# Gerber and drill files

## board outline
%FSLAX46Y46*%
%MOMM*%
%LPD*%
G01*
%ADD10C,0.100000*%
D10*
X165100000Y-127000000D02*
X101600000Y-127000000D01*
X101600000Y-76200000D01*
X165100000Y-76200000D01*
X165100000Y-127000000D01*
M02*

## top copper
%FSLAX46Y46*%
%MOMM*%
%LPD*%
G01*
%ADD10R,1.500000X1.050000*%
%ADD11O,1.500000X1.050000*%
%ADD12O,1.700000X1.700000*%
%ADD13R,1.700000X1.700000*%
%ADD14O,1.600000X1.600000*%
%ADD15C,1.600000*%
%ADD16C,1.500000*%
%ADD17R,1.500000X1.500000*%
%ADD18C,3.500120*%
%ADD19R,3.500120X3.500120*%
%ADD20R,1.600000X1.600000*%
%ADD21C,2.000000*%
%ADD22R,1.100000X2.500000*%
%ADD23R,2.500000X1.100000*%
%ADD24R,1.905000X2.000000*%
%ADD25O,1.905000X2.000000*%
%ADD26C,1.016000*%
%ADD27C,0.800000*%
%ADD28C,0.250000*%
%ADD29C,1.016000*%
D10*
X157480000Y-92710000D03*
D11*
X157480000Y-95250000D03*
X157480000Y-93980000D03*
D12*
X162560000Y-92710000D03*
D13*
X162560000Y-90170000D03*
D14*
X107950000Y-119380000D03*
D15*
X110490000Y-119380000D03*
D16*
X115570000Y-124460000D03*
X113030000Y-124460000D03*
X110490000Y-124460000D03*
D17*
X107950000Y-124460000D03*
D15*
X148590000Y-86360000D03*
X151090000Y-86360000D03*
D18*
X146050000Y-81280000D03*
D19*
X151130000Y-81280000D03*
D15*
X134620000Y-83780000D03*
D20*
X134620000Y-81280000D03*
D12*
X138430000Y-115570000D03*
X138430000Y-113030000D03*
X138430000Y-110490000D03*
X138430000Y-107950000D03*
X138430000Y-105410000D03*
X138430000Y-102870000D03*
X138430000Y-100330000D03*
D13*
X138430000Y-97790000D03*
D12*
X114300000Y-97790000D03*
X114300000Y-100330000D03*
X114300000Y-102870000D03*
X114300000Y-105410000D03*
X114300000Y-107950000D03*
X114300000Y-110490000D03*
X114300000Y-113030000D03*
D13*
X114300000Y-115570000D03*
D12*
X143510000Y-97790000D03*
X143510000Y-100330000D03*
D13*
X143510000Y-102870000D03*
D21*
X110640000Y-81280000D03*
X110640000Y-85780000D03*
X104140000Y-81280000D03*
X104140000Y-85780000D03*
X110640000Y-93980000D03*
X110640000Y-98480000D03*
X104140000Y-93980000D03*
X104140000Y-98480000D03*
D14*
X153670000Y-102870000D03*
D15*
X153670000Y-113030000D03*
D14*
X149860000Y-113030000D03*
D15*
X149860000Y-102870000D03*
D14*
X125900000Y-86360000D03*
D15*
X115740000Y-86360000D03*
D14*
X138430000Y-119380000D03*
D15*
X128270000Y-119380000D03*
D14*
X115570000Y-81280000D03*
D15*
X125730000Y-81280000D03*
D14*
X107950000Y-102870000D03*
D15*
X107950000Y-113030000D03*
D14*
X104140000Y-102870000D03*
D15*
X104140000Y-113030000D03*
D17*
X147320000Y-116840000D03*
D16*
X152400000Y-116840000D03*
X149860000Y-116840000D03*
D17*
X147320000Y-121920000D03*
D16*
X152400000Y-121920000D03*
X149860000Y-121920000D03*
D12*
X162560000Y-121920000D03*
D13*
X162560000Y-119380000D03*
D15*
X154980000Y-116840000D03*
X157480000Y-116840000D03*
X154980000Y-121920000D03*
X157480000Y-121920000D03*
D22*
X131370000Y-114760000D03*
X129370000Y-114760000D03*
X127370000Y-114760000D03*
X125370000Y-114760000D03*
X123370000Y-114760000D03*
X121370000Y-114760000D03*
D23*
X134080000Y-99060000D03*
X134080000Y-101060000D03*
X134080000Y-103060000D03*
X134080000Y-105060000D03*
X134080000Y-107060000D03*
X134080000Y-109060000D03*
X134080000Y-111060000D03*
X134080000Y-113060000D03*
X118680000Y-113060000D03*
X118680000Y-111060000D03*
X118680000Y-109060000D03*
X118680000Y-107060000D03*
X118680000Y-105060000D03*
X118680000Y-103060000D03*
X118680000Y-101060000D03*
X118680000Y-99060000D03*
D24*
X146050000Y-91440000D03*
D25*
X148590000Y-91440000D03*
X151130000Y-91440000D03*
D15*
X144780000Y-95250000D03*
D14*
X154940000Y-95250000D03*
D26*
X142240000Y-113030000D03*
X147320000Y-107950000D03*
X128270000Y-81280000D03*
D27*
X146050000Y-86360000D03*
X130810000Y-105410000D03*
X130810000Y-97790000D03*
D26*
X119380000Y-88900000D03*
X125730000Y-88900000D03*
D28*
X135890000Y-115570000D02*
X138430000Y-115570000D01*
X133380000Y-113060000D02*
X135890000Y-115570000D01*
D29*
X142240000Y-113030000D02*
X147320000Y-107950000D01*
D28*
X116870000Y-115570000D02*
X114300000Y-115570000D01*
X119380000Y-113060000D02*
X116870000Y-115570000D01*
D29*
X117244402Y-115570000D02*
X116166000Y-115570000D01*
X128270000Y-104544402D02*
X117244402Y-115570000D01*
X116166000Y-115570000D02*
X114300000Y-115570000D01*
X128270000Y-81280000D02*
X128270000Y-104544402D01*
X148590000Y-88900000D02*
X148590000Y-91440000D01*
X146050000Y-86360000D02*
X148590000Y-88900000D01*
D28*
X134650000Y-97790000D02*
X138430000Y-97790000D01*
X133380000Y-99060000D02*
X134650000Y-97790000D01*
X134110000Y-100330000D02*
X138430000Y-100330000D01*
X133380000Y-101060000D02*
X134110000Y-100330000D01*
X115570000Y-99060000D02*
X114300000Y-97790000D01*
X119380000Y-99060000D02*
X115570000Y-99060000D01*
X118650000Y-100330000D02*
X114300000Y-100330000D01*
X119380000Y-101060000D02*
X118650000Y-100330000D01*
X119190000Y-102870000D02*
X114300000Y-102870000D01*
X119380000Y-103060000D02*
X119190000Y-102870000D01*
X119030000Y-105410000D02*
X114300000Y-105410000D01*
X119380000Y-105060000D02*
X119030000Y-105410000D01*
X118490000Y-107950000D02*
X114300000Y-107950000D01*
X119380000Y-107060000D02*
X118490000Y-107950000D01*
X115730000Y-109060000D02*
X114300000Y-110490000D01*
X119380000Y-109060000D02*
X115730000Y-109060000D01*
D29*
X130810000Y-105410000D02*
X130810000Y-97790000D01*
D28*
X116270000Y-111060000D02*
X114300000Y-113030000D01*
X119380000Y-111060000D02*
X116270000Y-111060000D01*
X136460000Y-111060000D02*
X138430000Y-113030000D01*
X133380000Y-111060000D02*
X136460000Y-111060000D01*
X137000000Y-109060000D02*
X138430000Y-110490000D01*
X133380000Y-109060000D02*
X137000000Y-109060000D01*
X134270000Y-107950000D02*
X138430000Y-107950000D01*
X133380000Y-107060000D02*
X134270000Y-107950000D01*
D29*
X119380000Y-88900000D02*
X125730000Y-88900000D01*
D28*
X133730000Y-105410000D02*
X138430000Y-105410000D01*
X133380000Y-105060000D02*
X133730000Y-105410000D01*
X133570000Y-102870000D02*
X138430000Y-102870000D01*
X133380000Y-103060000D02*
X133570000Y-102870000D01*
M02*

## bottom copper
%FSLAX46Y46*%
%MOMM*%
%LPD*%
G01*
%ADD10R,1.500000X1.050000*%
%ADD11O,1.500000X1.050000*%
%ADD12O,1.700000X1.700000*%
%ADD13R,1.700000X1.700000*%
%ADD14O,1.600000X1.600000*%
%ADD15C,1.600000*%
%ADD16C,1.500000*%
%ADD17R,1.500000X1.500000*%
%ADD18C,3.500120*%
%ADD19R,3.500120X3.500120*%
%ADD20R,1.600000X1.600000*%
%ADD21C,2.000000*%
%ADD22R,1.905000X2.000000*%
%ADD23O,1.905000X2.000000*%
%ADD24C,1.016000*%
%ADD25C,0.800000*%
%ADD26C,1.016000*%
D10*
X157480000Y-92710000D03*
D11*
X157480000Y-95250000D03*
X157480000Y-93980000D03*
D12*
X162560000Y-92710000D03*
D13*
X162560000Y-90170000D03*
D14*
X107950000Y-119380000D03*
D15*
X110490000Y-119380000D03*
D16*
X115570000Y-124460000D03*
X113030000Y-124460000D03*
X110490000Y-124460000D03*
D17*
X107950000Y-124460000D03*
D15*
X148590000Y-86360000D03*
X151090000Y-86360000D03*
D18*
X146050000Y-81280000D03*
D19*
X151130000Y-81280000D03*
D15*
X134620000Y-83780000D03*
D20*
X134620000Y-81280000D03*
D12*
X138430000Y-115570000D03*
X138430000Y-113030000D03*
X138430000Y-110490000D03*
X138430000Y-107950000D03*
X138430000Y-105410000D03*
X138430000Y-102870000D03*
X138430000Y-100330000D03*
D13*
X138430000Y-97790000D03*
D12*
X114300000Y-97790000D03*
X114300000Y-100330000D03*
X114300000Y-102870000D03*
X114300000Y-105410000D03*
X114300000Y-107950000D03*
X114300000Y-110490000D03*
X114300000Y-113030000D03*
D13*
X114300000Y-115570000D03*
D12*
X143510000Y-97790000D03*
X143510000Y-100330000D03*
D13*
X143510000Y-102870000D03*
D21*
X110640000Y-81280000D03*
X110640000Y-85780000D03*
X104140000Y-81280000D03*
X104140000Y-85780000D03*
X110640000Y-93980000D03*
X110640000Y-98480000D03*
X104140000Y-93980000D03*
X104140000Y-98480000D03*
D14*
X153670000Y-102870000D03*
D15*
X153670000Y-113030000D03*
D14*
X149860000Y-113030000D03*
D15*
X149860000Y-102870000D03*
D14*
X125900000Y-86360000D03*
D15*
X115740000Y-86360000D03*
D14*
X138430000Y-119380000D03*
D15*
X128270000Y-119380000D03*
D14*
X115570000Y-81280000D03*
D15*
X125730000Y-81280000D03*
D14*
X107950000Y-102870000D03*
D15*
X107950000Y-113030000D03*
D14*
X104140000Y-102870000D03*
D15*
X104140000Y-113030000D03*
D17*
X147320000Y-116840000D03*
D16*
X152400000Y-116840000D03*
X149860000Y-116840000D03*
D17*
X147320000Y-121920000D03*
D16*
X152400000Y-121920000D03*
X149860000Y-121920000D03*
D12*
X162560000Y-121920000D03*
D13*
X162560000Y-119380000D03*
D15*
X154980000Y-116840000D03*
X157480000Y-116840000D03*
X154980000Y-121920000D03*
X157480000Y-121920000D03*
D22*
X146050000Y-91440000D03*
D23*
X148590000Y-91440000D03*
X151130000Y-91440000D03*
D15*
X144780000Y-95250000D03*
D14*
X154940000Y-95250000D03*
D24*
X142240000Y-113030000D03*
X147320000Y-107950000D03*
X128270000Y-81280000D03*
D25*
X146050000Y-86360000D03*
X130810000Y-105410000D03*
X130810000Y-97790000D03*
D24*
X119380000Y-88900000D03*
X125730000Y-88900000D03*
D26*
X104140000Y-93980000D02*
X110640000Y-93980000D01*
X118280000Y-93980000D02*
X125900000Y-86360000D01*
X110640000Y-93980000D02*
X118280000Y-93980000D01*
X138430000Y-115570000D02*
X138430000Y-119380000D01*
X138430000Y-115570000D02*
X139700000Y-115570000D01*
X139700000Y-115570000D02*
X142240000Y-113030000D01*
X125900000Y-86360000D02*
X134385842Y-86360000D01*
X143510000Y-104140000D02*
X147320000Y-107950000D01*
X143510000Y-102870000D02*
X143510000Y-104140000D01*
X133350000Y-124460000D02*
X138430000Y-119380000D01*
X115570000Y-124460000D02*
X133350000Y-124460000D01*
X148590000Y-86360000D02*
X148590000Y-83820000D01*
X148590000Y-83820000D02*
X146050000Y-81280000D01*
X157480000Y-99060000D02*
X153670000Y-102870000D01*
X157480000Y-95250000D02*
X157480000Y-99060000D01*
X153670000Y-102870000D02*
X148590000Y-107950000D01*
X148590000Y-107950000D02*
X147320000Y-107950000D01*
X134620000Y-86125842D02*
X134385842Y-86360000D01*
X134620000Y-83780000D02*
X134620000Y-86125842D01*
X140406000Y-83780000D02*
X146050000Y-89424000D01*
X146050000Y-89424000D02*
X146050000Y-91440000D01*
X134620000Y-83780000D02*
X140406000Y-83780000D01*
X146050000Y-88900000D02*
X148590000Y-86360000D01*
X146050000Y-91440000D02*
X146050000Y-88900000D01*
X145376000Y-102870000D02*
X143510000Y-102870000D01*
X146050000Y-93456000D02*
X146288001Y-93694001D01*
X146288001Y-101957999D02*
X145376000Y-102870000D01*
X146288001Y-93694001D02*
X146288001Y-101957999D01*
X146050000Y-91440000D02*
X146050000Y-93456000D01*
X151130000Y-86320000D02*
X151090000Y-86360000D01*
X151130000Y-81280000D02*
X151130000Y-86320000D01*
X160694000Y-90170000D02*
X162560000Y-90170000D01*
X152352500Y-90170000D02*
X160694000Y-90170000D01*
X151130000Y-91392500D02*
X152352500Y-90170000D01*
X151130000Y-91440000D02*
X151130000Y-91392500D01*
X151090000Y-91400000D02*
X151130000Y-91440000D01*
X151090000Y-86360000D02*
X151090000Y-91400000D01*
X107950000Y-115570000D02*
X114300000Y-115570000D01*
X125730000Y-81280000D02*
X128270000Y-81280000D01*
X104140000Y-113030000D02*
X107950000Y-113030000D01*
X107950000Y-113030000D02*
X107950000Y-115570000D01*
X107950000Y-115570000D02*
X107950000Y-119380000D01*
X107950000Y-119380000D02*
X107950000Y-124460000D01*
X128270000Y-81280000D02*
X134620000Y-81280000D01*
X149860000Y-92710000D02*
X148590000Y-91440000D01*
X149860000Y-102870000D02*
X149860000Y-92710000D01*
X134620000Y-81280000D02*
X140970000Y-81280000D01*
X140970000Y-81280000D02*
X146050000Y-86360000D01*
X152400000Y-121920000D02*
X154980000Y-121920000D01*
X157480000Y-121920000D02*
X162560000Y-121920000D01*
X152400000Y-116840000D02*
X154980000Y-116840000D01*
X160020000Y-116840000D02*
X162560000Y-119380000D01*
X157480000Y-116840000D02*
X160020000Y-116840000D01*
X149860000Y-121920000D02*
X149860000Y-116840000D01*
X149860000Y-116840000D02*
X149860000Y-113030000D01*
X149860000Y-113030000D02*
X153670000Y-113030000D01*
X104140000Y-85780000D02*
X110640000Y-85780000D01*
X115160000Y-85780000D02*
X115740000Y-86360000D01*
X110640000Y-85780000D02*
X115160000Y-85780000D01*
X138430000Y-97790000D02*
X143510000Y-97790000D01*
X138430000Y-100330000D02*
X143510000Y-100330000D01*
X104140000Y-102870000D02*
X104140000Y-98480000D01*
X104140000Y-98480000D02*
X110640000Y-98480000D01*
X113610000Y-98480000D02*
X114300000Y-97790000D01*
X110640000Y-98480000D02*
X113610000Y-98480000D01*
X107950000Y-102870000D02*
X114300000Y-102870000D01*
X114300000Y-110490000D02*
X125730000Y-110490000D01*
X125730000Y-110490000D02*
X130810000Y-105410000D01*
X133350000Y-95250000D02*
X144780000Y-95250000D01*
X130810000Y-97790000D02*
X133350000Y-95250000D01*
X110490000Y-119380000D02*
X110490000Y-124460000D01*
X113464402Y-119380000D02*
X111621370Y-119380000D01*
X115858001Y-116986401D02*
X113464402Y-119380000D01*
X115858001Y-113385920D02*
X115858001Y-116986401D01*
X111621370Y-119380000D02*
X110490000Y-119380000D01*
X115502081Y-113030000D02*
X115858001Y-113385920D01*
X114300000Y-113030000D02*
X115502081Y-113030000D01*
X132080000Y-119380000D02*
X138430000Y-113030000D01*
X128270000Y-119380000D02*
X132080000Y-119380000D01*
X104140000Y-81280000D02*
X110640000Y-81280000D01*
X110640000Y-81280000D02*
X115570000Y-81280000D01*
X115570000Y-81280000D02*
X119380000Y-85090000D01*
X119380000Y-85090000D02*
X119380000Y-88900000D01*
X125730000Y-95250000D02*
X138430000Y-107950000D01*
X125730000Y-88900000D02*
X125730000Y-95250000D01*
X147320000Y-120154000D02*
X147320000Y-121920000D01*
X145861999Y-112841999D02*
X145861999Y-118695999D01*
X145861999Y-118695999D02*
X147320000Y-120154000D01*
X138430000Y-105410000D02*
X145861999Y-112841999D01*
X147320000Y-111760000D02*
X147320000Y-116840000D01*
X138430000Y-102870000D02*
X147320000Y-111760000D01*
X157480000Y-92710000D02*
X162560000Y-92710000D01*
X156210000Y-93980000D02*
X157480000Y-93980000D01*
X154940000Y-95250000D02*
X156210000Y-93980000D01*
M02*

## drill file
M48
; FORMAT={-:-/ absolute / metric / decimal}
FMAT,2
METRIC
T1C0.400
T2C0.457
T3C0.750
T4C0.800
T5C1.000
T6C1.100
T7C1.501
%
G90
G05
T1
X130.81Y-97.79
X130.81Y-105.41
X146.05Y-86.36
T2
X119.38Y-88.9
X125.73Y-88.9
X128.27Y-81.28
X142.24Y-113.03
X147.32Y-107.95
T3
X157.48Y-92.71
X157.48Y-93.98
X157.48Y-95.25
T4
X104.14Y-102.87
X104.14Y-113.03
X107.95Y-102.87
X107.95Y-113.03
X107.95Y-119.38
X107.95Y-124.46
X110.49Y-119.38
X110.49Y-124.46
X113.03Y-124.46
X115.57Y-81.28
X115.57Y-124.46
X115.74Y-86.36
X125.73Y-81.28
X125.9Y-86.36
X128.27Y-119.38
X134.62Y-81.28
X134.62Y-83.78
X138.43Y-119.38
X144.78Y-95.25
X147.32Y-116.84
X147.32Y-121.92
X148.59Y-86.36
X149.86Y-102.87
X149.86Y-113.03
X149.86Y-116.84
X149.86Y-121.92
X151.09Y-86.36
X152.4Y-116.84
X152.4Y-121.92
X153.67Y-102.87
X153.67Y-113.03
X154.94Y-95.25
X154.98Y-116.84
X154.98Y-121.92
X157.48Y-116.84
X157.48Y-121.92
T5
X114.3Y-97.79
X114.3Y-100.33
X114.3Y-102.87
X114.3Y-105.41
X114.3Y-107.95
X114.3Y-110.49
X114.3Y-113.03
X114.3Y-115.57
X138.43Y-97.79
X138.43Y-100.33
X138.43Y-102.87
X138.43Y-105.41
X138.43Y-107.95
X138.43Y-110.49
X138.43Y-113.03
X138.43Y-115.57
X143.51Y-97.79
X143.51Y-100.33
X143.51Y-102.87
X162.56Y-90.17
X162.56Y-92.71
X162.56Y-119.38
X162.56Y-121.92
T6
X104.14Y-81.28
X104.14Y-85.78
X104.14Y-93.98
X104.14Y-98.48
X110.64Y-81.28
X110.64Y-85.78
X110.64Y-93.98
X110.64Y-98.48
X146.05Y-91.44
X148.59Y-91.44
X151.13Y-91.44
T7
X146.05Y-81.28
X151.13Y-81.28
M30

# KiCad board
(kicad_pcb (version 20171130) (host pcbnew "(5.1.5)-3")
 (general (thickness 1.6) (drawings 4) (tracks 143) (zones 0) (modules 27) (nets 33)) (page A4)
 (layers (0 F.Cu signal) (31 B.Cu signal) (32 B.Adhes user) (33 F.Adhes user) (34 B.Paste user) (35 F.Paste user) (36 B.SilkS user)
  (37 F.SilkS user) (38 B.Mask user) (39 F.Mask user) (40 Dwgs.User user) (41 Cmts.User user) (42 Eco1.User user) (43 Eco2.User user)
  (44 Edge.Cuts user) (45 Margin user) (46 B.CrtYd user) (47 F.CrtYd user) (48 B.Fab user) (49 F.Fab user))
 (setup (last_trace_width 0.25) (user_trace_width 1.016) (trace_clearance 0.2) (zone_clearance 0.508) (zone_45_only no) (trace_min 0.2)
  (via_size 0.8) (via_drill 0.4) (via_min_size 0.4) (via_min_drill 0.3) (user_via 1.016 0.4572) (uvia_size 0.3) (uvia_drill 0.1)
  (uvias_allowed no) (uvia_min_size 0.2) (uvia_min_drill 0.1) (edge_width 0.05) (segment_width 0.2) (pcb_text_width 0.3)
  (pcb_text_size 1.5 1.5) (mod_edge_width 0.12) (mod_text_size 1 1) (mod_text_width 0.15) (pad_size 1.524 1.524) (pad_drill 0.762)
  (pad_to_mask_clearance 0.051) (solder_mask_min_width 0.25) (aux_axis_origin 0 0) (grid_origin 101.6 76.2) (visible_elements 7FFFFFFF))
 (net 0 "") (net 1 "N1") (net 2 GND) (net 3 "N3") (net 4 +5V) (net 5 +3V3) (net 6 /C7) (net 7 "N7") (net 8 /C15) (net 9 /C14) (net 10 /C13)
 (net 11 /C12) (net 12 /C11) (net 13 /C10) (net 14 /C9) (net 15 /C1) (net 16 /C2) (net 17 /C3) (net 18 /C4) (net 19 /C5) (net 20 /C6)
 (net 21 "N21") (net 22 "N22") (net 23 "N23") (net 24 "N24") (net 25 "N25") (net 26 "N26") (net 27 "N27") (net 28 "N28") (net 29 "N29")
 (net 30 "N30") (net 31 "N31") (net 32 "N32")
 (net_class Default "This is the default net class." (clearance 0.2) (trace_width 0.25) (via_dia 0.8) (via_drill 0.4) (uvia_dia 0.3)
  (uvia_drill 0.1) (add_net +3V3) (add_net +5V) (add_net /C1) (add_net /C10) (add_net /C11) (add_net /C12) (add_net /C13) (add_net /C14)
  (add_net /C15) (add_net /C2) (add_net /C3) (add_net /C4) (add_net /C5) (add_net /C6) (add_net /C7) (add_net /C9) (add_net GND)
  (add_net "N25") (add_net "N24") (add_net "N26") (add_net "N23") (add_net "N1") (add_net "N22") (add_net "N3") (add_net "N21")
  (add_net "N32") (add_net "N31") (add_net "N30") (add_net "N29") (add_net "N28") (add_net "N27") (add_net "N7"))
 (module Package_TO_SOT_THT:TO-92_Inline (layer F.Cu) (at 157.48 92.71 270)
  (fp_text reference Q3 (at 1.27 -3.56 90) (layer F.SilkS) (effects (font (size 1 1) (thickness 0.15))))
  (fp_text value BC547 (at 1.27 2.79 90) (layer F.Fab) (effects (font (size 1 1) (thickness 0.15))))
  (pad 1 thru_hole rect (at 0 0 270) (size 1.05 1.5) (drill 0.75) (layers *.Cu *.Mask) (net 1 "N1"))
  (pad 3 thru_hole oval (at 2.54 0 270) (size 1.05 1.5) (drill 0.75) (layers *.Cu *.Mask) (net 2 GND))
  (pad 2 thru_hole oval (at 1.27 0 270) (size 1.05 1.5) (drill 0.75) (layers *.Cu *.Mask) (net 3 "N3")))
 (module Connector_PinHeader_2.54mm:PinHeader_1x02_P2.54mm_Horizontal (layer F.Cu) (at 162.56 90.17)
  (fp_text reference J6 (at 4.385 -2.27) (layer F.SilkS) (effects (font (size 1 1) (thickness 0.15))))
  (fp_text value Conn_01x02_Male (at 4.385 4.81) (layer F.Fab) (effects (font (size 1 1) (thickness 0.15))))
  (pad 2 thru_hole oval (at 0 2.54) (size 1.7 1.7) (drill 1) (layers *.Cu *.Mask) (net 1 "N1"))
  (pad 1 thru_hole rect (at 0 0) (size 1.7 1.7) (drill 1) (layers *.Cu *.Mask) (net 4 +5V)))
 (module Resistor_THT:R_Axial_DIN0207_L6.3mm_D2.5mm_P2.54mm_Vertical (layer F.Cu) (at 110.49 119.38 180)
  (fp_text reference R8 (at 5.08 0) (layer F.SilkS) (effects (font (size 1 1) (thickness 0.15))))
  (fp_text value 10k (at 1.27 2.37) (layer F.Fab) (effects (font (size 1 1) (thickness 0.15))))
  (pad 2 thru_hole oval (at 2.54 0 180) (size 1.6 1.6) (drill 0.8) (layers *.Cu *.Mask) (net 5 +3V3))
  (pad 1 thru_hole circle (at 0 0 180) (size 1.6 1.6) (drill 0.8) (layers *.Cu *.Mask) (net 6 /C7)))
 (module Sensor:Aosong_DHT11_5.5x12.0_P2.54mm (layer F.Cu) (at 107.95 124.46 90)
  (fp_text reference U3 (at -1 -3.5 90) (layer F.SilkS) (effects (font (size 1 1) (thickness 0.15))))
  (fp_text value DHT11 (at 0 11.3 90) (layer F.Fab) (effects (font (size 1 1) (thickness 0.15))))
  (pad 4 thru_hole circle (at 0 7.62 90) (size 1.5 1.5) (drill 0.8) (layers *.Cu *.Mask) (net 2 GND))
  (pad 3 thru_hole circle (at 0 5.08 90) (size 1.5 1.5) (drill 0.8) (layers *.Cu *.Mask) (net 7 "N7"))
  (pad 2 thru_hole circle (at 0 2.54 90) (size 1.5 1.5) (drill 0.8) (layers *.Cu *.Mask) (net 6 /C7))
  (pad 1 thru_hole rect (at 0 0 90) (size 1.5 1.5) (drill 0.8) (layers *.Cu *.Mask) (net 5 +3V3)))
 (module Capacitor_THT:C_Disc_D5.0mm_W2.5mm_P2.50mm (layer F.Cu) (at 151.09 86.36 180)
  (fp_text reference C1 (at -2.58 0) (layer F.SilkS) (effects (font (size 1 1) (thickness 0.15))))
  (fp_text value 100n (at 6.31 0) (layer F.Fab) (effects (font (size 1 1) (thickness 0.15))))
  (pad 2 thru_hole circle (at 2.5 0 180) (size 1.6 1.6) (drill 0.8) (layers *.Cu *.Mask) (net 2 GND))
  (pad 1 thru_hole circle (at 0 0 180) (size 1.6 1.6) (drill 0.8) (layers *.Cu *.Mask) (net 4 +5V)))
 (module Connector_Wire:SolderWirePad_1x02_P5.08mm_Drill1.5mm (layer F.Cu) (at 151.13 81.28 180)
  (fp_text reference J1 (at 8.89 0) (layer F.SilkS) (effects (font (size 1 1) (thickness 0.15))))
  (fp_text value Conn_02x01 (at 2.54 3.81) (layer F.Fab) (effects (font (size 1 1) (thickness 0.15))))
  (pad 2 thru_hole circle (at 5.08 0 180) (size 3.50012 3.50012) (drill 1.50114) (layers *.Cu *.Mask) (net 2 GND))
  (pad 1 thru_hole rect (at 0 0 180) (size 3.50012 3.50012) (drill 1.50114) (layers *.Cu *.Mask) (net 4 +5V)))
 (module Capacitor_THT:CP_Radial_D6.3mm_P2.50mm (layer F.Cu) (at 134.62 81.28 270)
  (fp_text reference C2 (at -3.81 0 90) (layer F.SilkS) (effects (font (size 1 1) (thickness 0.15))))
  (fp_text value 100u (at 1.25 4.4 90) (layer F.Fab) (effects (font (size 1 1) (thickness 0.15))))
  (pad 2 thru_hole circle (at 2.5 0 270) (size 1.6 1.6) (drill 0.8) (layers *.Cu *.Mask) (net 2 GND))
  (pad 1 thru_hole rect (at 0 0 270) (size 1.6 1.6) (drill 0.8) (layers *.Cu *.Mask) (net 5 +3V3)))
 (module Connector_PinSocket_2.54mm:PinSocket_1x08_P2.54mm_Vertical (layer F.Cu) (at 138.43 97.79)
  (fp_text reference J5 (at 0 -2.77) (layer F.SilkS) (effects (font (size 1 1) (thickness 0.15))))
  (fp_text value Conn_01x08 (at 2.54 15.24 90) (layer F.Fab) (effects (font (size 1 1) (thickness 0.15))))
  (pad 8 thru_hole oval (at 0 17.78) (size 1.7 1.7) (drill 1) (layers *.Cu *.Mask) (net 2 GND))
  (pad 7 thru_hole oval (at 0 15.24) (size 1.7 1.7) (drill 1) (layers *.Cu *.Mask) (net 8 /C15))
  (pad 6 thru_hole oval (at 0 12.7) (size 1.7 1.7) (drill 1) (layers *.Cu *.Mask) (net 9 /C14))
  (pad 5 thru_hole oval (at 0 10.16) (size 1.7 1.7) (drill 1) (layers *.Cu *.Mask) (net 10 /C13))
  (pad 4 thru_hole oval (at 0 7.62) (size 1.7 1.7) (drill 1) (layers *.Cu *.Mask) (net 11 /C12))
  (pad 3 thru_hole oval (at 0 5.08) (size 1.7 1.7) (drill 1) (layers *.Cu *.Mask) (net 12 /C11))
  (pad 2 thru_hole oval (at 0 2.54) (size 1.7 1.7) (drill 1) (layers *.Cu *.Mask) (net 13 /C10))
  (pad 1 thru_hole rect (at 0 0) (size 1.7 1.7) (drill 1) (layers *.Cu *.Mask) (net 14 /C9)))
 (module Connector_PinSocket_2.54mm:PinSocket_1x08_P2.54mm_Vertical (layer F.Cu) (at 114.3 115.57 180)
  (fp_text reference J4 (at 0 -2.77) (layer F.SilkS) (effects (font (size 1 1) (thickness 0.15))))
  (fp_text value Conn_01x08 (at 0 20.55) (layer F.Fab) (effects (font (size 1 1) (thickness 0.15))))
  (pad 8 thru_hole oval (at 0 17.78 180) (size 1.7 1.7) (drill 1) (layers *.Cu *.Mask) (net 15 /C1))
  (pad 7 thru_hole oval (at 0 15.24 180) (size 1.7 1.7) (drill 1) (layers *.Cu *.Mask) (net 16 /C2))
  (pad 6 thru_hole oval (at 0 12.7 180) (size 1.7 1.7) (drill 1) (layers *.Cu *.Mask) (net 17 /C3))
  (pad 5 thru_hole oval (at 0 10.16 180) (size 1.7 1.7) (drill 1) (layers *.Cu *.Mask) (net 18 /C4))
  (pad 4 thru_hole oval (at 0 7.62 180) (size 1.7 1.7) (drill 1) (layers *.Cu *.Mask) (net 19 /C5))
  (pad 3 thru_hole oval (at 0 5.08 180) (size 1.7 1.7) (drill 1) (layers *.Cu *.Mask) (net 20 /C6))
  (pad 2 thru_hole oval (at 0 2.54 180) (size 1.7 1.7) (drill 1) (layers *.Cu *.Mask) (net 6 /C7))
  (pad 1 thru_hole rect (at 0 0 180) (size 1.7 1.7) (drill 1) (layers *.Cu *.Mask) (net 5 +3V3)))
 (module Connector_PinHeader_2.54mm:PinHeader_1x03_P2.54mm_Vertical (layer F.Cu) (at 143.51 102.87 180)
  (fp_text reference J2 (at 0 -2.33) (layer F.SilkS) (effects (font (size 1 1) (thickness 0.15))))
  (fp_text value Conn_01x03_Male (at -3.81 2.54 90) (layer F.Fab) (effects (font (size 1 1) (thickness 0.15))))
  (pad 3 thru_hole oval (at 0 5.08 180) (size 1.7 1.7) (drill 1) (layers *.Cu *.Mask) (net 14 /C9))
  (pad 2 thru_hole oval (at 0 2.54 180) (size 1.7 1.7) (drill 1) (layers *.Cu *.Mask) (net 13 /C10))
  (pad 1 thru_hole rect (at 0 0 180) (size 1.7 1.7) (drill 1) (layers *.Cu *.Mask) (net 2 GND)))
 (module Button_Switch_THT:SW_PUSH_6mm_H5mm (layer F.Cu) (at 104.14 81.28)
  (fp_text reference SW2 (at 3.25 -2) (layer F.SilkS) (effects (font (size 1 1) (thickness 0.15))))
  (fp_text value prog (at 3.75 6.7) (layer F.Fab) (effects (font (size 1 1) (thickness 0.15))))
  (pad 1 thru_hole circle (at 6.5 0 90) (size 2 2) (drill 1.1) (layers *.Cu *.Mask) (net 10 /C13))
  (pad 2 thru_hole circle (at 6.5 4.5 90) (size 2 2) (drill 1.1) (layers *.Cu *.Mask) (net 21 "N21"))
  (pad 1 thru_hole circle (at 0 0 90) (size 2 2) (drill 1.1) (layers *.Cu *.Mask) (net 10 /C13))
  (pad 2 thru_hole circle (at 0 4.5 90) (size 2 2) (drill 1.1) (layers *.Cu *.Mask) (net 21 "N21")))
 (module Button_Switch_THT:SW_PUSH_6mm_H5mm (layer F.Cu) (at 104.14 93.98)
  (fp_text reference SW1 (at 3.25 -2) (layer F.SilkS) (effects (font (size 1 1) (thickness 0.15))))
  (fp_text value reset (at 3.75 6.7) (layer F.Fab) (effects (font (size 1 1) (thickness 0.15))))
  (pad 1 thru_hole circle (at 6.5 0 90) (size 2 2) (drill 1.1) (layers *.Cu *.Mask) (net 2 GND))
  (pad 2 thru_hole circle (at 6.5 4.5 90) (size 2 2) (drill 1.1) (layers *.Cu *.Mask) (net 15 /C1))
  (pad 1 thru_hole circle (at 0 0 90) (size 2 2) (drill 1.1) (layers *.Cu *.Mask) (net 2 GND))
  (pad 2 thru_hole circle (at 0 4.5 90) (size 2 2) (drill 1.1) (layers *.Cu *.Mask) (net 15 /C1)))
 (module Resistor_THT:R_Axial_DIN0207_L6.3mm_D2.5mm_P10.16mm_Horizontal (layer F.Cu) (at 153.67 113.03 90)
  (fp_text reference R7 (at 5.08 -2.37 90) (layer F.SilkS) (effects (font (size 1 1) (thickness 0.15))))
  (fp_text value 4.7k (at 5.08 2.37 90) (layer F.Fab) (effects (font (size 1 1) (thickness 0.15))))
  (pad 2 thru_hole oval (at 10.16 0 90) (size 1.6 1.6) (drill 0.8) (layers *.Cu *.Mask) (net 2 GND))
  (pad 1 thru_hole circle (at 0 0 90) (size 1.6 1.6) (drill 0.8) (layers *.Cu *.Mask) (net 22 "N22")))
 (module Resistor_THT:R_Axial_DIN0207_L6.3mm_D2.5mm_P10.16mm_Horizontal (layer F.Cu) (at 149.86 102.87 270)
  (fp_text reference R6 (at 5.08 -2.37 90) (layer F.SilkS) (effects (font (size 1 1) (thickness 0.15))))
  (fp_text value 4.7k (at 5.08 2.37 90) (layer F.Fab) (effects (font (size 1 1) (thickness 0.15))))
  (pad 2 thru_hole oval (at 10.16 0 270) (size 1.6 1.6) (drill 0.8) (layers *.Cu *.Mask) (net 22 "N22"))
  (pad 1 thru_hole circle (at 0 0 270) (size 1.6 1.6) (drill 0.8) (layers *.Cu *.Mask) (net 5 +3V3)))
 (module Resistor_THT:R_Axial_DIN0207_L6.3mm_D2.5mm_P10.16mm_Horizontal (layer F.Cu) (at 115.74 86.36)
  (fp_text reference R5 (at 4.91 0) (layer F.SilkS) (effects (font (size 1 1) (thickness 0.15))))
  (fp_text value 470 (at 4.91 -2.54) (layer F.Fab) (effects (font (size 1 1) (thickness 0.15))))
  (pad 2 thru_hole oval (at 10.16 0) (size 1.6 1.6) (drill 0.8) (layers *.Cu *.Mask) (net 2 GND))
  (pad 1 thru_hole circle (at 0 0) (size 1.6 1.6) (drill 0.8) (layers *.Cu *.Mask) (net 21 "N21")))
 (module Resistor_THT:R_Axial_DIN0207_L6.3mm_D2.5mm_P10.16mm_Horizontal (layer F.Cu) (at 128.27 119.38)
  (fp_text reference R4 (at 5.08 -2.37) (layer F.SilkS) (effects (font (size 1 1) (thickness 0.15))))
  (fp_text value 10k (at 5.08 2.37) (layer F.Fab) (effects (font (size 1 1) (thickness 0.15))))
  (pad 2 thru_hole oval (at 10.16 0) (size 1.6 1.6) (drill 0.8) (layers *.Cu *.Mask) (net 2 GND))
  (pad 1 thru_hole circle (at 0 0) (size 1.6 1.6) (drill 0.8) (layers *.Cu *.Mask) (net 8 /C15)))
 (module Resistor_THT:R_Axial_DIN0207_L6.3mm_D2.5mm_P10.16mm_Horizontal (layer F.Cu) (at 125.73 81.28 180)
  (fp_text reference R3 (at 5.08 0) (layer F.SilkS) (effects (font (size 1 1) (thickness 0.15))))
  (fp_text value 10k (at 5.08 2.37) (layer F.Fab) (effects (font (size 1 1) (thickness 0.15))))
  (pad 2 thru_hole oval (at 10.16 0 180) (size 1.6 1.6) (drill 0.8) (layers *.Cu *.Mask) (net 10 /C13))
  (pad 1 thru_hole circle (at 0 0 180) (size 1.6 1.6) (drill 0.8) (layers *.Cu *.Mask) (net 5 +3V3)))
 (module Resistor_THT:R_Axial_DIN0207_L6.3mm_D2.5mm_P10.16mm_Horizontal (layer F.Cu) (at 107.95 113.03 90)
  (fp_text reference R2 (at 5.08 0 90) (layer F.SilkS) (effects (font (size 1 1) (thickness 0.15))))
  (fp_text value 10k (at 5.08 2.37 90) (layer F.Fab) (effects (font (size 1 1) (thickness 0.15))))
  (pad 2 thru_hole oval (at 10.16 0 90) (size 1.6 1.6) (drill 0.8) (layers *.Cu *.Mask) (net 17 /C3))
  (pad 1 thru_hole circle (at 0 0 90) (size 1.6 1.6) (drill 0.8) (layers *.Cu *.Mask) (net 5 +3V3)))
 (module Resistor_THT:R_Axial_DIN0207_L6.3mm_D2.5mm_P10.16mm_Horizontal (layer F.Cu) (at 104.14 113.03 90)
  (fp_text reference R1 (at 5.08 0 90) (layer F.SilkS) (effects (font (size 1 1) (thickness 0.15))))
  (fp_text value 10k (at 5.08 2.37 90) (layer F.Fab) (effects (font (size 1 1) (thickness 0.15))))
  (pad 2 thru_hole oval (at 10.16 0 90) (size 1.6 1.6) (drill 0.8) (layers *.Cu *.Mask) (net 15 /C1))
  (pad 1 thru_hole circle (at 0 0 90) (size 1.6 1.6) (drill 0.8) (layers *.Cu *.Mask) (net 5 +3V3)))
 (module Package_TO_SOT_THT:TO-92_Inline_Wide (layer F.Cu) (at 147.32 116.84)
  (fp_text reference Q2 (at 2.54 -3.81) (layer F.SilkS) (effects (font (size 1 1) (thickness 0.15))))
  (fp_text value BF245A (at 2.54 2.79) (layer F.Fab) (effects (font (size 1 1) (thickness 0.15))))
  (pad 1 thru_hole rect (at 0 0 90) (size 1.5 1.5) (drill 0.8) (layers *.Cu *.Mask) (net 12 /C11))
  (pad 3 thru_hole circle (at 5.08 0 90) (size 1.5 1.5) (drill 0.8) (layers *.Cu *.Mask) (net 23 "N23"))
  (pad 2 thru_hole circle (at 2.54 0 90) (size 1.5 1.5) (drill 0.8) (layers *.Cu *.Mask) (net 22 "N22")))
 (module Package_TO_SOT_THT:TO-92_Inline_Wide (layer F.Cu) (at 147.32 121.92)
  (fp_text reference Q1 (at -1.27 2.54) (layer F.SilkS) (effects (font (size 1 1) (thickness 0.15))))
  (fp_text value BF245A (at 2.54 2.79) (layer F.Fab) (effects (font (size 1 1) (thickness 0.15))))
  (pad 1 thru_hole rect (at 0 0 90) (size 1.5 1.5) (drill 0.8) (layers *.Cu *.Mask) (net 11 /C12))
  (pad 3 thru_hole circle (at 5.08 0 90) (size 1.5 1.5) (drill 0.8) (layers *.Cu *.Mask) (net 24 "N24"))
  (pad 2 thru_hole circle (at 2.54 0 90) (size 1.5 1.5) (drill 0.8) (layers *.Cu *.Mask) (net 22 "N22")))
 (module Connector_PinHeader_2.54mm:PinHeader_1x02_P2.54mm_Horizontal (layer F.Cu) (at 162.56 119.38)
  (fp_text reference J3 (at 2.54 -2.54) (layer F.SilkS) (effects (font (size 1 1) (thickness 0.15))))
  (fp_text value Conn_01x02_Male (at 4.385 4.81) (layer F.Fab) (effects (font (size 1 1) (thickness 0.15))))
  (pad 2 thru_hole oval (at 0 2.54) (size 1.7 1.7) (drill 1) (layers *.Cu *.Mask) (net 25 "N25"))
  (pad 1 thru_hole rect (at 0 0) (size 1.7 1.7) (drill 1) (layers *.Cu *.Mask) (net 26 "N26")))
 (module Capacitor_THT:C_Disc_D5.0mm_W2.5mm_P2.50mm (layer F.Cu) (at 157.48 116.84 180)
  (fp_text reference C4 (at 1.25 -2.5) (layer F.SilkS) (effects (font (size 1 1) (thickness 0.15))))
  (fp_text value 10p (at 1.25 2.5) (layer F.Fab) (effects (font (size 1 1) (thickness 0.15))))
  (pad 2 thru_hole circle (at 2.5 0 180) (size 1.6 1.6) (drill 0.8) (layers *.Cu *.Mask) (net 23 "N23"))
  (pad 1 thru_hole circle (at 0 0 180) (size 1.6 1.6) (drill 0.8) (layers *.Cu *.Mask) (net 26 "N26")))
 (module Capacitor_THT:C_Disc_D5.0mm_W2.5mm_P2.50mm (layer F.Cu) (at 157.48 121.92 180)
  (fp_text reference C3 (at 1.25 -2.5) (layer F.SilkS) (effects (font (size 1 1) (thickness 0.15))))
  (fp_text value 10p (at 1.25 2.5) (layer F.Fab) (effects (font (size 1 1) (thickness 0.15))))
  (pad 2 thru_hole circle (at 2.5 0 180) (size 1.6 1.6) (drill 0.8) (layers *.Cu *.Mask) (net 24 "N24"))
  (pad 1 thru_hole circle (at 0 0 180) (size 1.6 1.6) (drill 0.8) (layers *.Cu *.Mask) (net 25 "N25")))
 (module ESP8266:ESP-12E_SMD (layer F.Cu) (at 119.38 99.06)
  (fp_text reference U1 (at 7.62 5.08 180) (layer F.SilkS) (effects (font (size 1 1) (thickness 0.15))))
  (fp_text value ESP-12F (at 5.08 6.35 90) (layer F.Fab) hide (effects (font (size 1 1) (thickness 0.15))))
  (pad 22 smd rect (at 11.99 15 90) (size 2.5 1.1) (drill (offset -0.7 0)) (layers F.Cu F.Paste F.Mask) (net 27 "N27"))
  (pad 21 smd rect (at 9.99 15 90) (size 2.5 1.1) (drill (offset -0.7 0)) (layers F.Cu F.Paste F.Mask) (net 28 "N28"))
  (pad 20 smd rect (at 7.99 15 90) (size 2.5 1.1) (drill (offset -0.7 0)) (layers F.Cu F.Paste F.Mask) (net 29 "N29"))
  (pad 19 smd rect (at 5.99 15 90) (size 2.5 1.1) (drill (offset -0.7 0)) (layers F.Cu F.Paste F.Mask) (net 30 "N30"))
  (pad 18 smd rect (at 3.99 15 90) (size 2.5 1.1) (drill (offset -0.7 0)) (layers F.Cu F.Paste F.Mask) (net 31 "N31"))
  (pad 17 smd rect (at 1.99 15 90) (size 2.5 1.1) (drill (offset -0.7 0)) (layers F.Cu F.Paste F.Mask) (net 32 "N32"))
  (pad 16 smd rect (at 14 0) (size 2.5 1.1) (drill (offset 0.7 0)) (layers F.Cu F.Paste F.Mask) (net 14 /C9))
  (pad 15 smd rect (at 14 2) (size 2.5 1.1) (drill (offset 0.7 0)) (layers F.Cu F.Paste F.Mask) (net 13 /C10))
  (pad 14 smd rect (at 14 4) (size 2.5 1.1) (drill (offset 0.7 0)) (layers F.Cu F.Paste F.Mask) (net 12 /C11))
  (pad 13 smd rect (at 14 6) (size 2.5 1.1) (drill (offset 0.7 0)) (layers F.Cu F.Paste F.Mask) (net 11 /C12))
  (pad 12 smd rect (at 14 8) (size 2.5 1.1) (drill (offset 0.7 0)) (layers F.Cu F.Paste F.Mask) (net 10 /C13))
  (pad 11 smd rect (at 14 10) (size 2.5 1.1) (drill (offset 0.7 0)) (layers F.Cu F.Paste F.Mask) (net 9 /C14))
  (pad 10 smd rect (at 14 12) (size 2.5 1.1) (drill (offset 0.7 0)) (layers F.Cu F.Paste F.Mask) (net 8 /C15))
  (pad 9 smd rect (at 14 14) (size 2.5 1.1) (drill (offset 0.7 0)) (layers F.Cu F.Paste F.Mask) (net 2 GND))
  (pad 8 smd rect (at 0 14) (size 2.5 1.1) (drill (offset -0.7 0)) (layers F.Cu F.Paste F.Mask) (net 5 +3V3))
  (pad 7 smd rect (at 0 12) (size 2.5 1.1) (drill (offset -0.7 0)) (layers F.Cu F.Paste F.Mask) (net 6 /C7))
  (pad 6 smd rect (at 0 10) (size 2.5 1.1) (drill (offset -0.7 0)) (layers F.Cu F.Paste F.Mask) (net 20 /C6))
  (pad 5 smd rect (at 0 8) (size 2.5 1.1) (drill (offset -0.7 0)) (layers F.Cu F.Paste F.Mask) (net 19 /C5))
  (pad 4 smd rect (at 0 6) (size 2.5 1.1) (drill (offset -0.7 0)) (layers F.Cu F.Paste F.Mask) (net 18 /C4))
  (pad 3 smd rect (at 0 4) (size 2.5 1.1) (drill (offset -0.7 0)) (layers F.Cu F.Paste F.Mask) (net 17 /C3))
  (pad 2 smd rect (at 0 2) (size 2.5 1.1) (drill (offset -0.7 0)) (layers F.Cu F.Paste F.Mask) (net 16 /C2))
  (pad 1 smd rect (at 0 0) (size 2.5 1.1) (drill (offset -0.7 0)) (layers F.Cu F.Paste F.Mask) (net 15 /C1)))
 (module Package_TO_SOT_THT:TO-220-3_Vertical (layer F.Cu) (at 146.05 91.44)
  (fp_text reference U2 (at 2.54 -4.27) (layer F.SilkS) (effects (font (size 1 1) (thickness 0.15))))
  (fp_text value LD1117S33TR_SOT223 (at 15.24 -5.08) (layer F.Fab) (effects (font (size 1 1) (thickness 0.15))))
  (pad 1 thru_hole rect (at 0 0) (size 1.905 2) (drill 1.1) (layers *.Cu *.Mask) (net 2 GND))
  (pad 2 thru_hole oval (at 2.54 0) (size 1.905 2) (drill 1.1) (layers *.Cu *.Mask) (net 5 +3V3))
  (pad 3 thru_hole oval (at 5.08 0) (size 1.905 2) (drill 1.1) (layers *.Cu *.Mask) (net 4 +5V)))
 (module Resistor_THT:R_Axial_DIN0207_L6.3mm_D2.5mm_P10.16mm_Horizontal (layer F.Cu) (at 144.78 95.25)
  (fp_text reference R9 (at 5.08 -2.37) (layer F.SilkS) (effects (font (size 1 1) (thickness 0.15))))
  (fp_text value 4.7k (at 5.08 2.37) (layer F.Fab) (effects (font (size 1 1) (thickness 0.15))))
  (pad 1 thru_hole circle (at 0 0) (size 1.6 1.6) (drill 0.8) (layers *.Cu *.Mask) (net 20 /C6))
  (pad 2 thru_hole oval (at 10.16 0) (size 1.6 1.6) (drill 0.8) (layers *.Cu *.Mask) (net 3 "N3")))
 (gr_poly (pts (xy 165.1 127) (xy 101.6 127) (xy 101.6 76.2) (xy 165.1 76.2)) (layer Edge.Cuts) (width 0.1))
 (segment (start 135.89 115.57) (end 138.43 115.57) (width 0.25) (layer F.Cu) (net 2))
 (segment (start 133.38 113.06) (end 135.89 115.57) (width 0.25) (layer F.Cu) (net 2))
 (segment (start 104.14 93.98) (end 110.64 93.98) (width 1.016) (layer B.Cu) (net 2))
 (segment (start 118.28 93.98) (end 125.9 86.36) (width 1.016) (layer B.Cu) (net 2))
 (segment (start 110.64 93.98) (end 118.28 93.98) (width 1.016) (layer B.Cu) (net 2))
 (segment (start 138.43 115.57) (end 138.43 119.38) (width 1.016) (layer B.Cu) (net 2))
 (segment (start 138.43 115.57) (end 139.7 115.57) (width 1.016) (layer B.Cu) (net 2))
 (via (at 142.24 113.03) (size 1.016) (drill 0.4572) (layers F.Cu B.Cu) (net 2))
 (segment (start 139.7 115.57) (end 142.24 113.03) (width 1.016) (layer B.Cu) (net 2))
 (segment (start 142.24 113.03) (end 147.32 107.95) (width 1.016) (layer F.Cu) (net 2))
 (via (at 147.32 107.95) (size 1.016) (drill 0.4572) (layers F.Cu B.Cu) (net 2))
 (segment (start 125.9 86.36) (end 134.385842 86.36) (width 1.016) (layer B.Cu) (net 2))
 (segment (start 143.51 104.14) (end 147.32 107.95) (width 1.016) (layer B.Cu) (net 2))
 (segment (start 143.51 102.87) (end 143.51 104.14) (width 1.016) (layer B.Cu) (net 2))
 (segment (start 133.35 124.46) (end 138.43 119.38) (width 1.016) (layer B.Cu) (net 2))
 (segment (start 115.57 124.46) (end 133.35 124.46) (width 1.016) (layer B.Cu) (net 2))
 (segment (start 148.59 86.36) (end 148.59 83.82) (width 1.016) (layer B.Cu) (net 2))
 (segment (start 148.59 83.82) (end 146.05 81.28) (width 1.016) (layer B.Cu) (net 2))
 (segment (start 157.48 99.06) (end 153.67 102.87) (width 1.016) (layer B.Cu) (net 2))
 (segment (start 157.48 95.25) (end 157.48 99.06) (width 1.016) (layer B.Cu) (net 2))
 (segment (start 153.67 102.87) (end 148.59 107.95) (width 1.016) (layer B.Cu) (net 2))
 (segment (start 148.59 107.95) (end 147.32 107.95) (width 1.016) (layer B.Cu) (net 2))
 (segment (start 134.62 86.125842) (end 134.385842 86.36) (width 1.016) (layer B.Cu) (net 2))
 (segment (start 134.62 83.78) (end 134.62 86.125842) (width 1.016) (layer B.Cu) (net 2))
 (segment (start 140.406 83.78) (end 146.05 89.424) (width 1.016) (layer B.Cu) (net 2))
 (segment (start 146.05 89.424) (end 146.05 91.44) (width 1.016) (layer B.Cu) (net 2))
 (segment (start 134.62 83.78) (end 140.406 83.78) (width 1.016) (layer B.Cu) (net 2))
 (segment (start 146.05 88.9) (end 148.59 86.36) (width 1.016) (layer B.Cu) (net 2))
 (segment (start 146.05 91.44) (end 146.05 88.9) (width 1.016) (layer B.Cu) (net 2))
 (segment (start 145.376 102.87) (end 143.51 102.87) (width 1.016) (layer B.Cu) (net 2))
 (segment (start 146.05 93.456) (end 146.288001 93.694001) (width 1.016) (layer B.Cu) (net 2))
 (segment (start 146.288001 101.957999) (end 145.376 102.87) (width 1.016) (layer B.Cu) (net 2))
 (segment (start 146.288001 93.694001) (end 146.288001 101.957999) (width 1.016) (layer B.Cu) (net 2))
 (segment (start 146.05 91.44) (end 146.05 93.456) (width 1.016) (layer B.Cu) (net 2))
 (segment (start 151.13 86.32) (end 151.09 86.36) (width 1.016) (layer B.Cu) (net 4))
 (segment (start 151.13 81.28) (end 151.13 86.32) (width 1.016) (layer B.Cu) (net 4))
 (segment (start 160.694 90.17) (end 162.56 90.17) (width 1.016) (layer B.Cu) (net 4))
 (segment (start 152.3525 90.17) (end 160.694 90.17) (width 1.016) (layer B.Cu) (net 4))
 (segment (start 151.13 91.3925) (end 152.3525 90.17) (width 1.016) (layer B.Cu) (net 4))
 (segment (start 151.13 91.44) (end 151.13 91.3925) (width 1.016) (layer B.Cu) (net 4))
 (segment (start 151.09 91.4) (end 151.13 91.44) (width 1.016) (layer B.Cu) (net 4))
 (segment (start 151.09 86.36) (end 151.09 91.4) (width 1.016) (layer B.Cu) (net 4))
 (segment (start 116.87 115.57) (end 114.3 115.57) (width 0.25) (layer F.Cu) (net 5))
 (segment (start 119.38 113.06) (end 116.87 115.57) (width 0.25) (layer F.Cu) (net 5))
 (segment (start 107.95 115.57) (end 114.3 115.57) (width 1.016) (layer B.Cu) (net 5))
 (via (at 128.27 81.28) (size 1.016) (drill 0.4572) (layers F.Cu B.Cu) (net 5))
 (segment (start 125.73 81.28) (end 128.27 81.28) (width 1.016) (layer B.Cu) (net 5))
 (segment (start 117.244402 115.57) (end 116.166 115.57) (width 1.016) (layer F.Cu) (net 5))
 (segment (start 128.27 104.544402) (end 117.244402 115.57) (width 1.016) (layer F.Cu) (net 5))
 (segment (start 116.166 115.57) (end 114.3 115.57) (width 1.016) (layer F.Cu) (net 5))
 (segment (start 128.27 81.28) (end 128.27 104.544402) (width 1.016) (layer F.Cu) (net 5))
 (segment (start 104.14 113.03) (end 107.95 113.03) (width 1.016) (layer B.Cu) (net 5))
 (segment (start 107.95 113.03) (end 107.95 115.57) (width 1.016) (layer B.Cu) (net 5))
 (segment (start 107.95 115.57) (end 107.95 119.38) (width 1.016) (layer B.Cu) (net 5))
 (segment (start 107.95 119.38) (end 107.95 124.46) (width 1.016) (layer B.Cu) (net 5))
 (segment (start 128.27 81.28) (end 134.62 81.28) (width 1.016) (layer B.Cu) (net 5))
 (segment (start 149.86 92.71) (end 148.59 91.44) (width 1.016) (layer B.Cu) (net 5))
 (segment (start 149.86 102.87) (end 149.86 92.71) (width 1.016) (layer B.Cu) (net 5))
 (via (at 146.05 86.36) (size 0.8) (drill 0.4) (layers F.Cu B.Cu) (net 5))
 (segment (start 134.62 81.28) (end 140.97 81.28) (width 1.016) (layer B.Cu) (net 5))
 (segment (start 140.97 81.28) (end 146.05 86.36) (width 1.016) (layer B.Cu) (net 5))
 (segment (start 148.59 88.9) (end 148.59 91.44) (width 1.016) (layer F.Cu) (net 5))
 (segment (start 146.05 86.36) (end 148.59 88.9) (width 1.016) (layer F.Cu) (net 5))
 (segment (start 152.4 121.92) (end 154.98 121.92) (width 1.016) (layer B.Cu) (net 24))
 (segment (start 157.48 121.92) (end 162.56 121.92) (width 1.016) (layer B.Cu) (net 25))
 (segment (start 152.4 116.84) (end 154.98 116.84) (width 1.016) (layer B.Cu) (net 23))
 (segment (start 160.02 116.84) (end 162.56 119.38) (width 1.016) (layer B.Cu) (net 26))
 (segment (start 157.48 116.84) (end 160.02 116.84) (width 1.016) (layer B.Cu) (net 26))
 (segment (start 149.86 121.92) (end 149.86 116.84) (width 1.016) (layer B.Cu) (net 22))
 (segment (start 149.86 116.84) (end 149.86 113.03) (width 1.016) (layer B.Cu) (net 22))
 (segment (start 149.86 113.03) (end 153.67 113.03) (width 1.016) (layer B.Cu) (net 22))
 (segment (start 104.14 85.78) (end 110.64 85.78) (width 1.016) (layer B.Cu) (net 21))
 (segment (start 115.16 85.78) (end 115.74 86.36) (width 1.016) (layer B.Cu) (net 21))
 (segment (start 110.64 85.78) (end 115.16 85.78) (width 1.016) (layer B.Cu) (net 21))
 (segment (start 134.65 97.79) (end 138.43 97.79) (width 0.25) (layer F.Cu) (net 14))
 (segment (start 133.38 99.06) (end 134.65 97.79) (width 0.25) (layer F.Cu) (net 14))
 (segment (start 138.43 97.79) (end 143.51 97.79) (width 1.016) (layer B.Cu) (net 14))
 (segment (start 134.11 100.33) (end 138.43 100.33) (width 0.25) (layer F.Cu) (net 13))
 (segment (start 133.38 101.06) (end 134.11 100.33) (width 0.25) (layer F.Cu) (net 13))
 (segment (start 138.43 100.33) (end 143.51 100.33) (width 1.016) (layer B.Cu) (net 13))
 (segment (start 115.57 99.06) (end 114.3 97.79) (width 0.25) (layer F.Cu) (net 15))
 (segment (start 119.38 99.06) (end 115.57 99.06) (width 0.25) (layer F.Cu) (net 15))
 (segment (start 104.14 102.87) (end 104.14 98.48) (width 1.016) (layer B.Cu) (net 15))
 (segment (start 104.14 98.48) (end 110.64 98.48) (width 1.016) (layer B.Cu) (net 15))
 (segment (start 113.61 98.48) (end 114.3 97.79) (width 1.016) (layer B.Cu) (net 15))
 (segment (start 110.64 98.48) (end 113.61 98.48) (width 1.016) (layer B.Cu) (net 15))
 (segment (start 118.65 100.33) (end 114.3 100.33) (width 0.25) (layer F.Cu) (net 16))
 (segment (start 119.38 101.06) (end 118.65 100.33) (width 0.25) (layer F.Cu) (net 16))
 (segment (start 119.19 102.87) (end 114.3 102.87) (width 0.25) (layer F.Cu) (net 17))
 (segment (start 119.38 103.06) (end 119.19 102.87) (width 0.25) (layer F.Cu) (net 17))
 (segment (start 107.95 102.87) (end 114.3 102.87) (width 1.016) (layer B.Cu) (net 17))
 (segment (start 119.03 105.41) (end 114.3 105.41) (width 0.25) (layer F.Cu) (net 18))
 (segment (start 119.38 105.06) (end 119.03 105.41) (width 0.25) (layer F.Cu) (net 18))
 (segment (start 118.49 107.95) (end 114.3 107.95) (width 0.25) (layer F.Cu) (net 19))
 (segment (start 119.38 107.06) (end 118.49 107.95) (width 0.25) (layer F.Cu) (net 19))
 (segment (start 115.73 109.06) (end 114.3 110.49) (width 0.25) (layer F.Cu) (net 20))
 (segment (start 119.38 109.06) (end 115.73 109.06) (width 0.25) (layer F.Cu) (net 20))
 (via (at 130.81 105.41) (size 0.8) (drill 0.4) (layers F.Cu B.Cu) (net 20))
 (segment (start 114.3 110.49) (end 125.73 110.49) (width 1.016) (layer B.Cu) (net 20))
 (segment (start 125.73 110.49) (end 130.81 105.41) (width 1.016) (layer B.Cu) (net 20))
 (segment (start 130.81 105.41) (end 130.81 97.79) (width 1.016) (layer F.Cu) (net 20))
 (via (at 130.81 97.79) (size 0.8) (drill 0.4) (layers F.Cu B.Cu) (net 20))
 (segment (start 133.35 95.25) (end 144.78 95.25) (width 1.016) (layer B.Cu) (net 20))
 (segment (start 130.81 97.79) (end 133.35 95.25) (width 1.016) (layer B.Cu) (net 20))
 (segment (start 116.27 111.06) (end 114.3 113.03) (width 0.25) (layer F.Cu) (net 6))
 (segment (start 119.38 111.06) (end 116.27 111.06) (width 0.25) (layer F.Cu) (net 6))
 (segment (start 110.49 119.38) (end 110.49 124.46) (width 1.016) (layer B.Cu) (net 6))
 (segment (start 113.464402 119.38) (end 111.62137 119.38) (width 1.016) (layer B.Cu) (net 6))
 (segment (start 115.858001 116.986401) (end 113.464402 119.38) (width 1.016) (layer B.Cu) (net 6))
 (segment (start 115.858001 113.38592) (end 115.858001 116.986401) (width 1.016) (layer B.Cu) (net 6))
 (segment (start 111.62137 119.38) (end 110.49 119.38) (width 1.016) (layer B.Cu) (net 6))
 (segment (start 115.502081 113.03) (end 115.858001 113.38592) (width 1.016) (layer B.Cu) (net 6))
 (segment (start 114.3 113.03) (end 115.502081 113.03) (width 1.016) (layer B.Cu) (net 6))
 (segment (start 136.46 111.06) (end 138.43 113.03) (width 0.25) (layer F.Cu) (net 8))
 (segment (start 133.38 111.06) (end 136.46 111.06) (width 0.25) (layer F.Cu) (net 8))
 (segment (start 132.08 119.38) (end 138.43 113.03) (width 1.016) (layer B.Cu) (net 8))
 (segment (start 128.27 119.38) (end 132.08 119.38) (width 1.016) (layer B.Cu) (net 8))
 (segment (start 137 109.06) (end 138.43 110.49) (width 0.25) (layer F.Cu) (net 9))
 (segment (start 133.38 109.06) (end 137 109.06) (width 0.25) (layer F.Cu) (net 9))
 (segment (start 134.27 107.95) (end 138.43 107.95) (width 0.25) (layer F.Cu) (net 10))
 (segment (start 133.38 107.06) (end 134.27 107.95) (width 0.25) (layer F.Cu) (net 10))
 (segment (start 104.14 81.28) (end 110.64 81.28) (width 1.016) (layer B.Cu) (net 10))
 (segment (start 110.64 81.28) (end 115.57 81.28) (width 1.016) (layer B.Cu) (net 10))
 (segment (start 115.57 81.28) (end 119.38 85.09) (width 1.016) (layer B.Cu) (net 10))
 (via (at 119.38 88.9) (size 1.016) (drill 0.4572) (layers F.Cu B.Cu) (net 10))
 (segment (start 119.38 85.09) (end 119.38 88.9) (width 1.016) (layer B.Cu) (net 10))
 (segment (start 119.38 88.9) (end 125.73 88.9) (width 1.016) (layer F.Cu) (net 10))
 (via (at 125.73 88.9) (size 1.016) (drill 0.4572) (layers F.Cu B.Cu) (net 10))
 (segment (start 125.73 95.25) (end 138.43 107.95) (width 1.016) (layer B.Cu) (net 10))
 (segment (start 125.73 88.9) (end 125.73 95.25) (width 1.016) (layer B.Cu) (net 10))
 (segment (start 133.73 105.41) (end 138.43 105.41) (width 0.25) (layer F.Cu) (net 11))
 (segment (start 133.38 105.06) (end 133.73 105.41) (width 0.25) (layer F.Cu) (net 11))
 (segment (start 147.32 120.154) (end 147.32 121.92) (width 1.016) (layer B.Cu) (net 11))
 (segment (start 145.861999 112.841999) (end 145.861999 118.695999) (width 1.016) (layer B.Cu) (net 11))
 (segment (start 145.861999 118.695999) (end 147.32 120.154) (width 1.016) (layer B.Cu) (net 11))
 (segment (start 138.43 105.41) (end 145.861999 112.841999) (width 1.016) (layer B.Cu) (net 11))
 (segment (start 133.57 102.87) (end 138.43 102.87) (width 0.25) (layer F.Cu) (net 12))
 (segment (start 133.38 103.06) (end 133.57 102.87) (width 0.25) (layer F.Cu) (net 12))
 (segment (start 147.32 111.76) (end 147.32 116.84) (width 1.016) (layer B.Cu) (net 12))
 (segment (start 138.43 102.87) (end 147.32 111.76) (width 1.016) (layer B.Cu) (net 12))
 (segment (start 157.48 92.71) (end 162.56 92.71) (width 1.016) (layer B.Cu) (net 1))
 (segment (start 156.21 93.98) (end 157.48 93.98) (width 1.016) (layer B.Cu) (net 3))
 (segment (start 154.94 95.25) (end 156.21 93.98) (width 1.016) (layer B.Cu) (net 3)))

